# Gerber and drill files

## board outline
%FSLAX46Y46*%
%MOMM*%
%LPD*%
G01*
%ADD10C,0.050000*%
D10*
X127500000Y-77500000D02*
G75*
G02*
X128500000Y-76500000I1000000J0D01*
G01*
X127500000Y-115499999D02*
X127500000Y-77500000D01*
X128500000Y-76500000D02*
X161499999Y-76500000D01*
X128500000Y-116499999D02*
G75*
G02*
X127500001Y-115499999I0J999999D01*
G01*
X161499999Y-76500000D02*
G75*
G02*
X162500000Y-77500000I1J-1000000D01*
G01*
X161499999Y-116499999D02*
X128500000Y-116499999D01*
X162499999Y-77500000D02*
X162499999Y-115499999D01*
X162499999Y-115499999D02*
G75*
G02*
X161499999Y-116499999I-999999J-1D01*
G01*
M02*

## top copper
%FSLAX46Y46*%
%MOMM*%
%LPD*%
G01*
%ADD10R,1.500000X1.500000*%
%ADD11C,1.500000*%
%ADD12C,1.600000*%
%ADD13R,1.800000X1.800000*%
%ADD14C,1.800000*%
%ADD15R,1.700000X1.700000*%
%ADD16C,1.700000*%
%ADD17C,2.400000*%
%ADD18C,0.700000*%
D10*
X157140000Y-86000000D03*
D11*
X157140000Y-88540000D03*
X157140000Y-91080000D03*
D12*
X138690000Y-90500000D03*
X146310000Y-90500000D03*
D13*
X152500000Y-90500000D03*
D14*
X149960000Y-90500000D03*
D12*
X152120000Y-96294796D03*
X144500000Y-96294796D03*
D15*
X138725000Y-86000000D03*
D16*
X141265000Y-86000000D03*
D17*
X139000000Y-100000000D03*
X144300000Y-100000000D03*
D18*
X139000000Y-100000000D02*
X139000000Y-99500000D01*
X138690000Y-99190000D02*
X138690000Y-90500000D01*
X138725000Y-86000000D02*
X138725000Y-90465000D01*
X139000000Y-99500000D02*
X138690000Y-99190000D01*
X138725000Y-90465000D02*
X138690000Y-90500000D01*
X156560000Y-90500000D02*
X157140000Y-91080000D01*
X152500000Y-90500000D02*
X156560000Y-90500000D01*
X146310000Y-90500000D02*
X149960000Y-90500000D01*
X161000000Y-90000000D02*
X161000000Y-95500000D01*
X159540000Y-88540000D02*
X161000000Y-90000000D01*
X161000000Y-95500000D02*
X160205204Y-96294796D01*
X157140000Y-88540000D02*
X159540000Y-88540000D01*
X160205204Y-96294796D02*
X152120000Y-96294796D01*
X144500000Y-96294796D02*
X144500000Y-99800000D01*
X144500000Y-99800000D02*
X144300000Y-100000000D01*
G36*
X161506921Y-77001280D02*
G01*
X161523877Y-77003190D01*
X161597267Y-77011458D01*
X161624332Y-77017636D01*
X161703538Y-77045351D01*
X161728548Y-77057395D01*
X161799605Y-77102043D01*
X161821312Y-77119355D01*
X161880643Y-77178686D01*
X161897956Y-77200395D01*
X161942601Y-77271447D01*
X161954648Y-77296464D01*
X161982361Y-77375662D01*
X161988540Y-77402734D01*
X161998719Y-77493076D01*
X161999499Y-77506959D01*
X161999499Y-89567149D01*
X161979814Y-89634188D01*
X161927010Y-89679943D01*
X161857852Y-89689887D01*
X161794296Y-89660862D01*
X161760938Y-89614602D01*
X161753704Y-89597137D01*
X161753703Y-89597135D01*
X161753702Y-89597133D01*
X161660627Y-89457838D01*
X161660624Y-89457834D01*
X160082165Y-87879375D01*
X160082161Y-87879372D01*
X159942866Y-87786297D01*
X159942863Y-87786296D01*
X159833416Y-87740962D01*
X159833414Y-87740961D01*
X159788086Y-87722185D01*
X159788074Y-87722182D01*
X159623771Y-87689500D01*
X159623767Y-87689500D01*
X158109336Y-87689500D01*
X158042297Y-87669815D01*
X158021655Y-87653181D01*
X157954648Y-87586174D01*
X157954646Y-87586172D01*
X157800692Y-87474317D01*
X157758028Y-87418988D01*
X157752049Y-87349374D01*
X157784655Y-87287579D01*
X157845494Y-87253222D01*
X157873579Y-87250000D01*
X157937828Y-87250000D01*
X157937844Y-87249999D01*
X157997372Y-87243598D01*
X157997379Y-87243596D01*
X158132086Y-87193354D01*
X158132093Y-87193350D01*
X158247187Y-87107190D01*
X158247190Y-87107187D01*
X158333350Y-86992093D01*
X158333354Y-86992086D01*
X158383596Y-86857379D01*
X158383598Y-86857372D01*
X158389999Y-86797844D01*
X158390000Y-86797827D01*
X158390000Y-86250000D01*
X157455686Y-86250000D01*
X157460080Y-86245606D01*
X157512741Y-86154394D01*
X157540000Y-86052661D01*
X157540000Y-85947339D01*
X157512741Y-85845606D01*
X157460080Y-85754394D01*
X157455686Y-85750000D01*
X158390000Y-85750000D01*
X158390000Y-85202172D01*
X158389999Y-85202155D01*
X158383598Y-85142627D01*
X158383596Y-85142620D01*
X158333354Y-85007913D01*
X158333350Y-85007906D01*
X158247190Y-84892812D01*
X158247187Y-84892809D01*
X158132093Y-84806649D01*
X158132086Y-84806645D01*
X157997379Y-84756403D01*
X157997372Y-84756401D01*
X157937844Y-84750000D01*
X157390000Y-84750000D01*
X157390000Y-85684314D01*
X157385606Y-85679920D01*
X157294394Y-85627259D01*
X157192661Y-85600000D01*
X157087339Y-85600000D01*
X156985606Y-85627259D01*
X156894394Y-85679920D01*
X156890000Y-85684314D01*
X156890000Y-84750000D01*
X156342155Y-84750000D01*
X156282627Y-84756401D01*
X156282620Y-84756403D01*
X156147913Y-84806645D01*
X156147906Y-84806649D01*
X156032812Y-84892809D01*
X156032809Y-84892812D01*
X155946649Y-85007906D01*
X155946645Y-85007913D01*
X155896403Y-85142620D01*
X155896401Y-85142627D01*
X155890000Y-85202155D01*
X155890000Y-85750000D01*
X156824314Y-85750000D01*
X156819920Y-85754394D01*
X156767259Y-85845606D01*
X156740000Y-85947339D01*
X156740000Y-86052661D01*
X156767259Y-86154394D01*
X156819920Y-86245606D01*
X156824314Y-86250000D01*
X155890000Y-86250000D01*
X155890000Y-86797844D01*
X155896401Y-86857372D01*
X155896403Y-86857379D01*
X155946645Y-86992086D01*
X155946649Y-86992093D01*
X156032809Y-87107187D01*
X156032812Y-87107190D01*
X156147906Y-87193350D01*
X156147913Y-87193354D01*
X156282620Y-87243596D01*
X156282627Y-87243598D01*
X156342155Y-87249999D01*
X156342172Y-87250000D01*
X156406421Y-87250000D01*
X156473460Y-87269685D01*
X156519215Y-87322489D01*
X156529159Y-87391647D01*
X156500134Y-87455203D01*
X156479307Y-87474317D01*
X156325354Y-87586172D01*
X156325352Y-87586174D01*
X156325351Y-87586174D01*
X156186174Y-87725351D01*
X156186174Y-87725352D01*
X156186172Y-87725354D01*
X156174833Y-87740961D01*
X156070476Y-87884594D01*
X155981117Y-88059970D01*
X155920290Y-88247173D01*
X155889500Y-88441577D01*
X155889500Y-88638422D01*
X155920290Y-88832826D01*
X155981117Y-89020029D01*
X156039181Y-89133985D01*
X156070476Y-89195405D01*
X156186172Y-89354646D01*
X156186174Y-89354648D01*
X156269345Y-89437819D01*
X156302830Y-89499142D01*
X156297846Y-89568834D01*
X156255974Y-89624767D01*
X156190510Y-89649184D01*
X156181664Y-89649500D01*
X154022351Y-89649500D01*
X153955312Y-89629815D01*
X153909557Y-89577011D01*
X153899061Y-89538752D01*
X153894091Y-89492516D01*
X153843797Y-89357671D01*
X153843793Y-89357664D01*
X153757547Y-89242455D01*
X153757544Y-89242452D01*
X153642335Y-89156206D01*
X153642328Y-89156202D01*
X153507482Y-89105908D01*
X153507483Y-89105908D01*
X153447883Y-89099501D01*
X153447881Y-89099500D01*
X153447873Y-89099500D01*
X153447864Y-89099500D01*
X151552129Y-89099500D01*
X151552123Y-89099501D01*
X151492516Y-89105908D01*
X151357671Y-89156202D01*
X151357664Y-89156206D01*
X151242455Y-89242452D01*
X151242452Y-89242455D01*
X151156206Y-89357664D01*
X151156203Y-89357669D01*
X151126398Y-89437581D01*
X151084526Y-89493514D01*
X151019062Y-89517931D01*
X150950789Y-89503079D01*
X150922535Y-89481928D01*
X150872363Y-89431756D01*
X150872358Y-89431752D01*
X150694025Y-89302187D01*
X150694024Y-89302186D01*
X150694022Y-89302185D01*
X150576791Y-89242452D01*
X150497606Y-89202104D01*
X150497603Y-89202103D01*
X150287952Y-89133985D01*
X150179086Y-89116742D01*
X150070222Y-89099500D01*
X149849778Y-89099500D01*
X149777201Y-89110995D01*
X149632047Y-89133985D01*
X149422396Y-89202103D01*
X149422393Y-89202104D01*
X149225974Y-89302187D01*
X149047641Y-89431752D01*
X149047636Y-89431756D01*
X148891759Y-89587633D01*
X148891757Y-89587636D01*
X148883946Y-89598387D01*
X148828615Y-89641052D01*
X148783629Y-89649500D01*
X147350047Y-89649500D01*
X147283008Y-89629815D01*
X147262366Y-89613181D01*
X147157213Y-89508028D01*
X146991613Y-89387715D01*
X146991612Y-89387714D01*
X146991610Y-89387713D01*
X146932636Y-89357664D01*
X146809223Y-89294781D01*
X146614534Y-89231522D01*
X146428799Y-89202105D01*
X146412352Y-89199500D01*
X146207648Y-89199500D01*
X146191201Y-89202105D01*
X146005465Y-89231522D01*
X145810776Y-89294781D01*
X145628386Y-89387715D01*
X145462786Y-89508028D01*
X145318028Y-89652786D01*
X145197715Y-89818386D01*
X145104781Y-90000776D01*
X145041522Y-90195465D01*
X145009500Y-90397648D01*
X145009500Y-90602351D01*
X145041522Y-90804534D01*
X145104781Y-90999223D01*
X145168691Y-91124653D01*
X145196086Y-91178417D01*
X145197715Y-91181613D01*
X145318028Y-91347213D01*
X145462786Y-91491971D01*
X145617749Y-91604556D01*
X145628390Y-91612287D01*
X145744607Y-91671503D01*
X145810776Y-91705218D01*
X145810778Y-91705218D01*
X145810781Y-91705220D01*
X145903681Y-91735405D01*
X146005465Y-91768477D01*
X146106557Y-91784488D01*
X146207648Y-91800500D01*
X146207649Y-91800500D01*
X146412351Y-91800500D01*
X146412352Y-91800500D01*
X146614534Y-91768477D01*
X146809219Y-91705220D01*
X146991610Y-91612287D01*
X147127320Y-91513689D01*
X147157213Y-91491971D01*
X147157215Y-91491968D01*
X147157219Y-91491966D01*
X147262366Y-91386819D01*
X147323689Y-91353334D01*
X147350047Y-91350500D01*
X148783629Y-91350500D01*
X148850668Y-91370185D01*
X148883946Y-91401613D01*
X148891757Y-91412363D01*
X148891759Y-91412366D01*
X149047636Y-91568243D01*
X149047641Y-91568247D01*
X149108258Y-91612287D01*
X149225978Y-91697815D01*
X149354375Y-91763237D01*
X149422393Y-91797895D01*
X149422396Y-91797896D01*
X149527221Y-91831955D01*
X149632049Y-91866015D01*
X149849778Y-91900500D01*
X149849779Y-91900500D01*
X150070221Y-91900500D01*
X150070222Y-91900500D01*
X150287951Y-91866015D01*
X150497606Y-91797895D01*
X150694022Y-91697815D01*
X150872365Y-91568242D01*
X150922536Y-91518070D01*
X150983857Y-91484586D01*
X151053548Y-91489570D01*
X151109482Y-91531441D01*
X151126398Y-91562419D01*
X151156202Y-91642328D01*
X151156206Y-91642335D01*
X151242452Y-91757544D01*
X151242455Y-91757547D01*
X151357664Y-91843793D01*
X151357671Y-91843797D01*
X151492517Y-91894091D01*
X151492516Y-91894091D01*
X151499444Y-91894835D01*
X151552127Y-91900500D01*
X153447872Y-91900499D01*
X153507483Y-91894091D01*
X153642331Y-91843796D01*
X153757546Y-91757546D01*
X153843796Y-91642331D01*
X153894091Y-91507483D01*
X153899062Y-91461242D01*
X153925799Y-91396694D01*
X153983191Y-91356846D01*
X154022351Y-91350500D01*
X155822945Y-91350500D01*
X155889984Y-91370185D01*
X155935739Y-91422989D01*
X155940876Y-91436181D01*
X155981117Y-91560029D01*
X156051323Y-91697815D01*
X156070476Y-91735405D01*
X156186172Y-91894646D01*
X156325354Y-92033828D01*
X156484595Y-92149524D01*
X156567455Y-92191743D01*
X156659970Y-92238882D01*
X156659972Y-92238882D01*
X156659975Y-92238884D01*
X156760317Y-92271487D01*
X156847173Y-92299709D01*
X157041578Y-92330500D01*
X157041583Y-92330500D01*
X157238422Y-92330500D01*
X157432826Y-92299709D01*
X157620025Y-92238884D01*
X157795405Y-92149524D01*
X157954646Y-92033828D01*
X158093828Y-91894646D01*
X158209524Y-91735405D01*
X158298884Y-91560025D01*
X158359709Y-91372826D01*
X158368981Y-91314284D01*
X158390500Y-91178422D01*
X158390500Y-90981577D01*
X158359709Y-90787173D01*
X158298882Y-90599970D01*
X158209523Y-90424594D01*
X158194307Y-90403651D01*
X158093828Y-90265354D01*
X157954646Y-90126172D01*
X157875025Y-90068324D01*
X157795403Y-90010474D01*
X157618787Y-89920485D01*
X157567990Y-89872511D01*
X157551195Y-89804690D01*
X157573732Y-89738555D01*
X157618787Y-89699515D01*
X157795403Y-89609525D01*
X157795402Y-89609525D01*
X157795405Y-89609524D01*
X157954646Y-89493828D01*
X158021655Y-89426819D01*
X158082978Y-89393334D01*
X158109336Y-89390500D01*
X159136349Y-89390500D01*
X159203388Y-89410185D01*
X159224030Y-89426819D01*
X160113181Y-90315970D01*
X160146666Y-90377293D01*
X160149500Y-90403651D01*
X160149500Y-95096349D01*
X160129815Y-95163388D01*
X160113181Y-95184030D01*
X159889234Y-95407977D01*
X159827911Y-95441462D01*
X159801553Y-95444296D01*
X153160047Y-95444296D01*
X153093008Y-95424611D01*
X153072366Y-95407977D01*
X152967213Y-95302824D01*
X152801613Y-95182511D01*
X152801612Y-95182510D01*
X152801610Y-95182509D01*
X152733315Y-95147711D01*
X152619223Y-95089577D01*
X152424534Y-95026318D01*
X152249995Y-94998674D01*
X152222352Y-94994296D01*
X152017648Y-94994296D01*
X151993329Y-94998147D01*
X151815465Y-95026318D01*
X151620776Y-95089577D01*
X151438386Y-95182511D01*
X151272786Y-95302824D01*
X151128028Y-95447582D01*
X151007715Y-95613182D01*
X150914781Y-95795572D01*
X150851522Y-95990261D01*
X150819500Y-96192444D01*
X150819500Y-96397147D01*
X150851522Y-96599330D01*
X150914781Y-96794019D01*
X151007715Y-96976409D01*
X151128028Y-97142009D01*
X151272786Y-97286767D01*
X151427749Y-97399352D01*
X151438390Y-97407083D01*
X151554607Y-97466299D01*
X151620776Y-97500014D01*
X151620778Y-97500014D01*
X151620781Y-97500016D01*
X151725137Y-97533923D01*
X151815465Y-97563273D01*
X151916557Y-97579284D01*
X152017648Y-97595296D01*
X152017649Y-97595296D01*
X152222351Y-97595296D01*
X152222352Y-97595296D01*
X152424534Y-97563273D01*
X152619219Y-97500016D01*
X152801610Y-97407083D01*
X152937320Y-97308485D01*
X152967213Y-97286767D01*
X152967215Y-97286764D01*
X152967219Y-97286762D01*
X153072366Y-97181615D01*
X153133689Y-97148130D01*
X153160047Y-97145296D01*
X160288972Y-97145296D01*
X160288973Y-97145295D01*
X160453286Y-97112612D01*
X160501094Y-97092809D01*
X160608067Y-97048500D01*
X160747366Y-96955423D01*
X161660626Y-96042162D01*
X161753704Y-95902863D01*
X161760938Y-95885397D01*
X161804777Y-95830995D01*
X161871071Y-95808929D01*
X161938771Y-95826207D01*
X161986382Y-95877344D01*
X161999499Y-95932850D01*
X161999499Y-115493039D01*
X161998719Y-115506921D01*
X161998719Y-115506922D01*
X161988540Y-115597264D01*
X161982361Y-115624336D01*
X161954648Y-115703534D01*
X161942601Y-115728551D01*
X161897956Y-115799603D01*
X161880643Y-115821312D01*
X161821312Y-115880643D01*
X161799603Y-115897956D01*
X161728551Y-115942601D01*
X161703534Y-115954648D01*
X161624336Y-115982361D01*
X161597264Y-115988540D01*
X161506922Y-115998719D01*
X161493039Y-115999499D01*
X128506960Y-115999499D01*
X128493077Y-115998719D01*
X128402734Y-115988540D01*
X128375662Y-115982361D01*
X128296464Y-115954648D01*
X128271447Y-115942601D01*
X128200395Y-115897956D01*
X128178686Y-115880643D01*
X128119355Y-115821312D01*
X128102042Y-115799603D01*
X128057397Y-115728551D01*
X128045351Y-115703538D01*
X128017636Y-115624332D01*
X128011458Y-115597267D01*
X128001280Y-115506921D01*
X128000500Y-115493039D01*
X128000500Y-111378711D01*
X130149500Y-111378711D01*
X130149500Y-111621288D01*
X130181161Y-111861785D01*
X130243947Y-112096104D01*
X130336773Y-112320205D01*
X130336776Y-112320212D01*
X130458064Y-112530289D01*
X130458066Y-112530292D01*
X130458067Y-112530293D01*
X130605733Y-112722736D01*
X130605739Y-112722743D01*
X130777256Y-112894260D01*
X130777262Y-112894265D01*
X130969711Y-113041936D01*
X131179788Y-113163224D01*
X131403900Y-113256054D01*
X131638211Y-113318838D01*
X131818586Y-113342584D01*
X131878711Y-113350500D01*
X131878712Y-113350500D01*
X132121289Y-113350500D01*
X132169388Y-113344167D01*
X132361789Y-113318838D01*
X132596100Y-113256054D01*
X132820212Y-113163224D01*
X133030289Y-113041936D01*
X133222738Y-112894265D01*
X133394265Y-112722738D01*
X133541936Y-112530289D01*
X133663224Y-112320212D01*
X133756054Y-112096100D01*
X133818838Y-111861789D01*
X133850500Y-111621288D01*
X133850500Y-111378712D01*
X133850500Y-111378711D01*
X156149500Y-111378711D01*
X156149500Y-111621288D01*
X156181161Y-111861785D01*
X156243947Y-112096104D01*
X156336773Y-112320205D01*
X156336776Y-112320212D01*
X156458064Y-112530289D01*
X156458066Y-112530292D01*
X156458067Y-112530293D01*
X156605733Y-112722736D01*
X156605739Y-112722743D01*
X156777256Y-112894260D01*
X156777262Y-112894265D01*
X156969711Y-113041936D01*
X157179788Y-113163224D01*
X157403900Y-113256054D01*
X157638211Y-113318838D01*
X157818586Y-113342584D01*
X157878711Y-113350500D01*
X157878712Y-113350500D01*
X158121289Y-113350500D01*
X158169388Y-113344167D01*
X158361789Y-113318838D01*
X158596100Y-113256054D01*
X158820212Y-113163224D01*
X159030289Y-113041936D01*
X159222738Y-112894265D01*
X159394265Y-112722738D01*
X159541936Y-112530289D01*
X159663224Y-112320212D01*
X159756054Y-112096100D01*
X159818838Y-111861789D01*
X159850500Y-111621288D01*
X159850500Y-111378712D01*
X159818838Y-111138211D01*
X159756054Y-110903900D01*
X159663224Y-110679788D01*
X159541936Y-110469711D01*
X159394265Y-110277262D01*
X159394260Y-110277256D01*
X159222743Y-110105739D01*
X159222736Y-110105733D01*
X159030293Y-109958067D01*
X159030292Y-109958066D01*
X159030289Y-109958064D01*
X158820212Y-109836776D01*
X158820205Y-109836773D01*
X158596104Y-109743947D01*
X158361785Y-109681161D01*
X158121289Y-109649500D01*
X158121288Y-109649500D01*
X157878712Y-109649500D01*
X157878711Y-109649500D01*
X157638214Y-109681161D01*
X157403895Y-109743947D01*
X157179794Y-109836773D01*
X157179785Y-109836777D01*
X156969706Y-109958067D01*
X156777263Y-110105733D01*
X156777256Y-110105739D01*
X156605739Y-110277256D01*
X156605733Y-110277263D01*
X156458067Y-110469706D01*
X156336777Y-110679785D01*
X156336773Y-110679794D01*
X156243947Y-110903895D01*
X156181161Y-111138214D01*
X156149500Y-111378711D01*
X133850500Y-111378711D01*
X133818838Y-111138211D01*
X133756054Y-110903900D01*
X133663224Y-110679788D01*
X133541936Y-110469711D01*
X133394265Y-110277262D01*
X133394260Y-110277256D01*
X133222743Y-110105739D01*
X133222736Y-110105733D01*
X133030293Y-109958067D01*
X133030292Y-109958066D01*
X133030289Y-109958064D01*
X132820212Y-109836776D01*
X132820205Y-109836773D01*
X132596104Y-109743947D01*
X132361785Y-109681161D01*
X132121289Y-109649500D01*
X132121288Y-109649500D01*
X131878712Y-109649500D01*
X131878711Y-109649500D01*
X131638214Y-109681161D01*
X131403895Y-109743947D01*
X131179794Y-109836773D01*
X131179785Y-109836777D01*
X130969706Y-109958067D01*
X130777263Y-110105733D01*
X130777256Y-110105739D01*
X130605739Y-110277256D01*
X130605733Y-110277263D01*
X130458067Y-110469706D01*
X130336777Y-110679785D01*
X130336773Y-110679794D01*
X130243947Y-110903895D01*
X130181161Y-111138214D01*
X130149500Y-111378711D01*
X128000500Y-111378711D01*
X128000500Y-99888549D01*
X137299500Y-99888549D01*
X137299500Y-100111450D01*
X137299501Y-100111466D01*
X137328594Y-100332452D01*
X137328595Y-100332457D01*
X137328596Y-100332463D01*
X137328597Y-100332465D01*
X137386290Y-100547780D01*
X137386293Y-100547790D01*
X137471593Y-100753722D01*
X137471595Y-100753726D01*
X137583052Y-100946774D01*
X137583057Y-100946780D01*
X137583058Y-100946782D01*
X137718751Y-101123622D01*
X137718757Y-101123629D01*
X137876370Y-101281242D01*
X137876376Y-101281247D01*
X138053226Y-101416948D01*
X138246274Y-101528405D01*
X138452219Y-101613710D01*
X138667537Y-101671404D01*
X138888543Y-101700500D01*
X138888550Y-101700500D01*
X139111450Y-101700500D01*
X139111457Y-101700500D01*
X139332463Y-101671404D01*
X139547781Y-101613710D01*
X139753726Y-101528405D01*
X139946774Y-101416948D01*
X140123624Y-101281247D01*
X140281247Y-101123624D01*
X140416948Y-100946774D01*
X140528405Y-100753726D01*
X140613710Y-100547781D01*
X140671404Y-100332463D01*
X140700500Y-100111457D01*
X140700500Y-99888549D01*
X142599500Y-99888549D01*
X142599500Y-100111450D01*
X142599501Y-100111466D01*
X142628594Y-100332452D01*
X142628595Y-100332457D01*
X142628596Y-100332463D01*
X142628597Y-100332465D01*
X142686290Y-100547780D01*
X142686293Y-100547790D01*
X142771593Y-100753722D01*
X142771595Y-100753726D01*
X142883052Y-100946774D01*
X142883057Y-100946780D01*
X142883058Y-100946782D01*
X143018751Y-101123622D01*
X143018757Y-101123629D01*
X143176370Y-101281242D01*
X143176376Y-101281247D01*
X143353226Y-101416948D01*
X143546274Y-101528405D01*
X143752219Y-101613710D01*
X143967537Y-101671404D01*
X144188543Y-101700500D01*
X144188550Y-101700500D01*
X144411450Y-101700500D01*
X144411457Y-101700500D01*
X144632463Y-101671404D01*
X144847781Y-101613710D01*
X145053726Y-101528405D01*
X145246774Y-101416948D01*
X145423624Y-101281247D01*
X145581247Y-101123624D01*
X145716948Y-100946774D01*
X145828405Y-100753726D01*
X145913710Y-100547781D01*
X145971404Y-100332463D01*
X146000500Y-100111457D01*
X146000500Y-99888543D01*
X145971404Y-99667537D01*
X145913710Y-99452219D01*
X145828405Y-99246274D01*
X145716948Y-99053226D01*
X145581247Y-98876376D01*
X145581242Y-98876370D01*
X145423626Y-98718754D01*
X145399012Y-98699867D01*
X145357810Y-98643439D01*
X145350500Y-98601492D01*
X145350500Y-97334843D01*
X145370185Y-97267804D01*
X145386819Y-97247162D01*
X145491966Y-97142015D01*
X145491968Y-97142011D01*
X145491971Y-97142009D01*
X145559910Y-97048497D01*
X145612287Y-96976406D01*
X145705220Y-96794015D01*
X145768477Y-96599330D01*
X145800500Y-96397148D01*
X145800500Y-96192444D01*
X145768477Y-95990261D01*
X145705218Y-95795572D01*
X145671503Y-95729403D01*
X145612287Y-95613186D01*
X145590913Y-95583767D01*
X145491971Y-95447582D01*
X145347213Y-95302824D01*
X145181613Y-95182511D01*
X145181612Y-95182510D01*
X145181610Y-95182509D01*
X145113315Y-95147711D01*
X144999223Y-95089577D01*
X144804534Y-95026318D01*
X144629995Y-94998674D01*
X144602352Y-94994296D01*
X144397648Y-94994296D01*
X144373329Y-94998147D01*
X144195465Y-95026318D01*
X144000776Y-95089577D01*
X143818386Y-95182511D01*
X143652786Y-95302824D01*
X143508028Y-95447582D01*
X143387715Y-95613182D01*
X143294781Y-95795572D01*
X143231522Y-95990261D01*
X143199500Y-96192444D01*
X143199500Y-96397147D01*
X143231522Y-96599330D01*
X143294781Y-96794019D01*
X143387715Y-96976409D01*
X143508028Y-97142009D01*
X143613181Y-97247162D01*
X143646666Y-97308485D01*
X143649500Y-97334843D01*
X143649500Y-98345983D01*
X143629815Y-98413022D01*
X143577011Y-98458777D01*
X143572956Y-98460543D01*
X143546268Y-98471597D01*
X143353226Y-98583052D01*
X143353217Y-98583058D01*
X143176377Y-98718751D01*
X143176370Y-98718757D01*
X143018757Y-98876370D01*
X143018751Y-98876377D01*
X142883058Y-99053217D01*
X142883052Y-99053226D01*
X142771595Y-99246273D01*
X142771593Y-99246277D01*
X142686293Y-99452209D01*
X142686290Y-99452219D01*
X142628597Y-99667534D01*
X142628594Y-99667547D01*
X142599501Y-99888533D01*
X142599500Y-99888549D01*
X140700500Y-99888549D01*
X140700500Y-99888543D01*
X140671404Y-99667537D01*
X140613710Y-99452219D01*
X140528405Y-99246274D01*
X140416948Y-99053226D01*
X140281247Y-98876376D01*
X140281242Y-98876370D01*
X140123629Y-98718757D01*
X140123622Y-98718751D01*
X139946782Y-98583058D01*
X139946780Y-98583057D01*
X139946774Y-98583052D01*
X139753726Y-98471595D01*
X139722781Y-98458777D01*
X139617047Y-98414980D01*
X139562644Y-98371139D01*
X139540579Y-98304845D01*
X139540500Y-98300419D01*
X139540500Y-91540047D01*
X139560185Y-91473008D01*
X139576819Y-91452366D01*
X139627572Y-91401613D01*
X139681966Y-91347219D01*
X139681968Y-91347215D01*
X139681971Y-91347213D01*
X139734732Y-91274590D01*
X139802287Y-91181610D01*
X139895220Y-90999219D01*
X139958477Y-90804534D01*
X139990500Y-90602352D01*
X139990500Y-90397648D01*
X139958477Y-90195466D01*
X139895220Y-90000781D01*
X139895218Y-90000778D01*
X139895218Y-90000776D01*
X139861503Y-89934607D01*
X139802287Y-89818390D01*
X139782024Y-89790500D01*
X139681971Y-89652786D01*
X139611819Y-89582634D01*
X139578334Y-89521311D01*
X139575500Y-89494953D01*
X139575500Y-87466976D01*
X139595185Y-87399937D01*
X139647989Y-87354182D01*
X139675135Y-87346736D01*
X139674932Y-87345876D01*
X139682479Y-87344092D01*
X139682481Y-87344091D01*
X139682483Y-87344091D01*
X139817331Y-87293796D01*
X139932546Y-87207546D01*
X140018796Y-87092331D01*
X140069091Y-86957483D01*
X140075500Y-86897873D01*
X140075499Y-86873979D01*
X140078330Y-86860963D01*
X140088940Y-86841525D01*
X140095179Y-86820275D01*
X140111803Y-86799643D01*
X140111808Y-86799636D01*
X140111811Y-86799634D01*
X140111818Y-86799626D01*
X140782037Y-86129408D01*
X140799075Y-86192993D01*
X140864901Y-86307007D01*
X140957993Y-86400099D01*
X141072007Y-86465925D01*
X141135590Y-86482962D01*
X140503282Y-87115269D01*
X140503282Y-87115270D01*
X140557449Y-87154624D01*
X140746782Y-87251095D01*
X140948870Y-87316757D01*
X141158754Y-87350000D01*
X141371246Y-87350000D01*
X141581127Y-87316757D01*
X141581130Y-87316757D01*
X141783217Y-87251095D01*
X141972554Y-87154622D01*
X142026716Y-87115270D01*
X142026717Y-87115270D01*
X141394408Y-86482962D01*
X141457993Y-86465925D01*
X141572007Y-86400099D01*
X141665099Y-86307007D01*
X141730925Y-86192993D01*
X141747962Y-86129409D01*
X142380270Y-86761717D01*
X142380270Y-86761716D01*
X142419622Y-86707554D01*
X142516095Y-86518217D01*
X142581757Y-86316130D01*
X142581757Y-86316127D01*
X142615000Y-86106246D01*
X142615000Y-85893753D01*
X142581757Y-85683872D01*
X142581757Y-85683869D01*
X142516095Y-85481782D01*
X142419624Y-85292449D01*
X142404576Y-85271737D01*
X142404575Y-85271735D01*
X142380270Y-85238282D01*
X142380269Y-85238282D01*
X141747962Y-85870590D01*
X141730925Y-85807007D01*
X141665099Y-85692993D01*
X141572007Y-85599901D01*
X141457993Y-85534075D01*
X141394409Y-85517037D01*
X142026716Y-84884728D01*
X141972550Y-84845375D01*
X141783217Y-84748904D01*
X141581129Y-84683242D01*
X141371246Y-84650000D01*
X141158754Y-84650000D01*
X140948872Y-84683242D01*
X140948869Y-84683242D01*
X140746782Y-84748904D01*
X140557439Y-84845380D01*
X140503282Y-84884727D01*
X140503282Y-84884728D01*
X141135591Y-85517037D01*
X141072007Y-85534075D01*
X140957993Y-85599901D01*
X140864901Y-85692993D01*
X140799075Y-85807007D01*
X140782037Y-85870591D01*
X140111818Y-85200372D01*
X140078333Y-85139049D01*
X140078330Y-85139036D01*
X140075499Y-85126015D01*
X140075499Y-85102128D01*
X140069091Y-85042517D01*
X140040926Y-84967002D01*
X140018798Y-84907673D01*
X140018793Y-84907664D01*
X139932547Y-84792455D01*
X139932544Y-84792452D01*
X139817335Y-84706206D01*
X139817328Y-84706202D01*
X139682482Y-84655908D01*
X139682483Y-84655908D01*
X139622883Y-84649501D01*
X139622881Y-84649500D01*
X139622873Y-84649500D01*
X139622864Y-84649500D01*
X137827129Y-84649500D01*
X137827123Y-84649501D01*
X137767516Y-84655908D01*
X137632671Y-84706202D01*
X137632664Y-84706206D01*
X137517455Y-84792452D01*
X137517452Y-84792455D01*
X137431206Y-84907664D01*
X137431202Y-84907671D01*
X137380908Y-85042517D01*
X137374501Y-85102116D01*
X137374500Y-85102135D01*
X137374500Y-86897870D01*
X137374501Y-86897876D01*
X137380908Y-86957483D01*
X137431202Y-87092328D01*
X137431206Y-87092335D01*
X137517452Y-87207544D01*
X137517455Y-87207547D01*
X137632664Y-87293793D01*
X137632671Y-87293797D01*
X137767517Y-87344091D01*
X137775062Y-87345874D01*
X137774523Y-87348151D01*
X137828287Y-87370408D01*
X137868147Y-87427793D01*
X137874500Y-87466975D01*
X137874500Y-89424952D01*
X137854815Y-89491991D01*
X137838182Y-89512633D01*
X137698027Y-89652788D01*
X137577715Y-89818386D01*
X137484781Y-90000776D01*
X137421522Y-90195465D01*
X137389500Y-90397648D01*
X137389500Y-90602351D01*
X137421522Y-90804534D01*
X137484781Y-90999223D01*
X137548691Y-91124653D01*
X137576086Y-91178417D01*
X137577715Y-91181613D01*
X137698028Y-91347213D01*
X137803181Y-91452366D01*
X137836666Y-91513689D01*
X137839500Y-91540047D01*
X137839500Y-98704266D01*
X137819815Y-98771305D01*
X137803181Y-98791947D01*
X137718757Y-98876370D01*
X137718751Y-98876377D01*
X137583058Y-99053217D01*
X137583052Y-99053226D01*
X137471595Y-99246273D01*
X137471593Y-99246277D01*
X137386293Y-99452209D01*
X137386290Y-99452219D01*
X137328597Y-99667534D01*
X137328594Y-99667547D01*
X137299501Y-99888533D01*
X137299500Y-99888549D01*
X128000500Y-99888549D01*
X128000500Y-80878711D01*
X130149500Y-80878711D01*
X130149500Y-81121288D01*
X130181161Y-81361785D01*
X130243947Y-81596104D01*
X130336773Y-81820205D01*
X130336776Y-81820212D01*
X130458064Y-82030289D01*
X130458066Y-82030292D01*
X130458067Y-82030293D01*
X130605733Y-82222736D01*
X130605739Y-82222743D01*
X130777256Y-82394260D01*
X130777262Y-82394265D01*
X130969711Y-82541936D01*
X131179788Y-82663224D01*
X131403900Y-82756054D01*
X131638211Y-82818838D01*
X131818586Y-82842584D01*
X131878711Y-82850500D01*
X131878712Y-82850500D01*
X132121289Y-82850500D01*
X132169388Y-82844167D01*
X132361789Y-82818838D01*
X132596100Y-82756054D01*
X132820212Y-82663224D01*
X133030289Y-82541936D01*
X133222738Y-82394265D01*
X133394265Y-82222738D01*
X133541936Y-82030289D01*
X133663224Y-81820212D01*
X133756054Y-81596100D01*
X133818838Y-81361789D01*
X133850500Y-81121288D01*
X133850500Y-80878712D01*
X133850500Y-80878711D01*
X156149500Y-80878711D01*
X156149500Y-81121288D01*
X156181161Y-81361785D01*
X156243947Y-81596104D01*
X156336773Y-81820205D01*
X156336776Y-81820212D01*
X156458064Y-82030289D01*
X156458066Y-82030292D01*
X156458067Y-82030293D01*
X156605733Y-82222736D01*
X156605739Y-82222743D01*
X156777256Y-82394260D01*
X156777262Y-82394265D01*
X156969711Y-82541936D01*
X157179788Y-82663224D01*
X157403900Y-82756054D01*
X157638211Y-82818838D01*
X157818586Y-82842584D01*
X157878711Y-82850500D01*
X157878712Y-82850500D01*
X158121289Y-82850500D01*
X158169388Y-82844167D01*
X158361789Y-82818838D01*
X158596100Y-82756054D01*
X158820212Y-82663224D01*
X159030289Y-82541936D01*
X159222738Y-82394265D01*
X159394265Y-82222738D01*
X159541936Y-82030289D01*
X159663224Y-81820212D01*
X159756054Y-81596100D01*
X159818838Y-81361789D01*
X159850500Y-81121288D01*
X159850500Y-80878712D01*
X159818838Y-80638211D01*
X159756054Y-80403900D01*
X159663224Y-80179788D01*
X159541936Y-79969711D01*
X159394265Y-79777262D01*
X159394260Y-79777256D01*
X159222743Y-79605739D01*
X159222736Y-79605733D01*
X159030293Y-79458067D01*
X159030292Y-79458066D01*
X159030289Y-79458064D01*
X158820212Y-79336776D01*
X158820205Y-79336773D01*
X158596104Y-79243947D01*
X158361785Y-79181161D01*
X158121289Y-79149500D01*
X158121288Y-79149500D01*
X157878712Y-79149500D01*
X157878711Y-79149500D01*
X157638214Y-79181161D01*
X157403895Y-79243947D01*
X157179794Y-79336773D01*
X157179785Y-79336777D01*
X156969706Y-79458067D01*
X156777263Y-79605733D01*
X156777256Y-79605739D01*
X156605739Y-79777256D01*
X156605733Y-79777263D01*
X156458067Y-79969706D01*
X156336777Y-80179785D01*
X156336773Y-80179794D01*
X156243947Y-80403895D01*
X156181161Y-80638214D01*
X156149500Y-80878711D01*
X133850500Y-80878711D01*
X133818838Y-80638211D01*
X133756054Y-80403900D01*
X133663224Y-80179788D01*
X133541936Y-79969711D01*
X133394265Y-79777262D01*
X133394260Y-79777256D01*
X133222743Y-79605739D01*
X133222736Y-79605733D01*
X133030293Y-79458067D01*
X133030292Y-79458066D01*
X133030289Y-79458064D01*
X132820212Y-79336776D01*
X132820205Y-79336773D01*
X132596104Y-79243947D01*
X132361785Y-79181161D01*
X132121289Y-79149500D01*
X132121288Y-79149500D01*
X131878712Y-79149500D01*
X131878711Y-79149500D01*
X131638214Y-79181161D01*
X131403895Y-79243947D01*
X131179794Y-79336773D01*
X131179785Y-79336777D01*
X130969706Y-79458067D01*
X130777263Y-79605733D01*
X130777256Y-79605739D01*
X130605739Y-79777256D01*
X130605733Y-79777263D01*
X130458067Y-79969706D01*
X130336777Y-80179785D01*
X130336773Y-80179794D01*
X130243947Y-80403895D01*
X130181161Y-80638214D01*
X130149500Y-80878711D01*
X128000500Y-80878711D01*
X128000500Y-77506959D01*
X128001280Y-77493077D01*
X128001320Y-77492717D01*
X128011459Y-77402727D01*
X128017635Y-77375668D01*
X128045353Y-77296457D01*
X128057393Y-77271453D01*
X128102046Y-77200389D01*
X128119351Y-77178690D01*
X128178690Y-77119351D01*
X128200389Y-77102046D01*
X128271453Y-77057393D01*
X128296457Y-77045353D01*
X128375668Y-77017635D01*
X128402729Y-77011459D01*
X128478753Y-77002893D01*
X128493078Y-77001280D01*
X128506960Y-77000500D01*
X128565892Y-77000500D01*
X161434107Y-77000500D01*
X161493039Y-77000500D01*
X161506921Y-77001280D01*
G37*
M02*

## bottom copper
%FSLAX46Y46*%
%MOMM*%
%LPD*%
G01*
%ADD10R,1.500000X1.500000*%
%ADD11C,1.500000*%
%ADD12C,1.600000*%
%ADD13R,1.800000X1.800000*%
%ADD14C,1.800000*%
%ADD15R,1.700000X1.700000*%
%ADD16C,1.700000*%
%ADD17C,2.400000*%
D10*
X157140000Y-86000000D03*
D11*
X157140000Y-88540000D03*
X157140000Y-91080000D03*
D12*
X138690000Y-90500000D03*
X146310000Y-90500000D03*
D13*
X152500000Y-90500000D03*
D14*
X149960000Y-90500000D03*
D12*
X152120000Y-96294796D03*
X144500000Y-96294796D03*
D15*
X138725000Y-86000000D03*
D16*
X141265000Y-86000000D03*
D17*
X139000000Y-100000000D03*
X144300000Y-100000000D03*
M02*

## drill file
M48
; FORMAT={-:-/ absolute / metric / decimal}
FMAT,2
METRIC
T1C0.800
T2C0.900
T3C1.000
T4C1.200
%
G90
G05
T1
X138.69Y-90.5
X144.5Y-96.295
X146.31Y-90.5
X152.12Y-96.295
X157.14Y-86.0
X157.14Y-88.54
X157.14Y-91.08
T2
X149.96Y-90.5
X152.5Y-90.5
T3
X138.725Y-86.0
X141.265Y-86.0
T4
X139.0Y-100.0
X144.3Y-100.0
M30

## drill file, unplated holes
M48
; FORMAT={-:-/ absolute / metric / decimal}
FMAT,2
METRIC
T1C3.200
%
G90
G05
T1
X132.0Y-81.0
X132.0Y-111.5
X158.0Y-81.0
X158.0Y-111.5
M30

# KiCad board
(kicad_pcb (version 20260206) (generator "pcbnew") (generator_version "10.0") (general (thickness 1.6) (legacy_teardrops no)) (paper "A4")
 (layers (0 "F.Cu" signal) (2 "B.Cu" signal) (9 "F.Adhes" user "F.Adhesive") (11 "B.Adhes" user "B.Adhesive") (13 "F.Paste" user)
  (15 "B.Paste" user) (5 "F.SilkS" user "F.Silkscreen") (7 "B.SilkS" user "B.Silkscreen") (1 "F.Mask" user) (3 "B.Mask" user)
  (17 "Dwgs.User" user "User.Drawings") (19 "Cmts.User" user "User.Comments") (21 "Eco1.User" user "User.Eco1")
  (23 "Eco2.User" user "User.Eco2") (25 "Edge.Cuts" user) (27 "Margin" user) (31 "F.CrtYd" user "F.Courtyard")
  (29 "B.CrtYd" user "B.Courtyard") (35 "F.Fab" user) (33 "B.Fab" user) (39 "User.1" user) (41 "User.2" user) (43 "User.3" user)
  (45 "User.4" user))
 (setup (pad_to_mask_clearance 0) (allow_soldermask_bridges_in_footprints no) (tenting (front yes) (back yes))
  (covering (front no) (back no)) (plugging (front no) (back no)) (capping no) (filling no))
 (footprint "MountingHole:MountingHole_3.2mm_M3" (layer "F.Cu") (at 132 81)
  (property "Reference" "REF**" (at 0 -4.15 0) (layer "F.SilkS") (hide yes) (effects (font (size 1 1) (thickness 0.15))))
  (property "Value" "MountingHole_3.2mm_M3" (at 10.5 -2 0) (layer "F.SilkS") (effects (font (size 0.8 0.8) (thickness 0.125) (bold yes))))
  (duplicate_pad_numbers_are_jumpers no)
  (pad "" np_thru_hole circle (at 0 0) (size 3.2 3.2) (drill 3.2) (layers "*.Cu" "*.Mask")))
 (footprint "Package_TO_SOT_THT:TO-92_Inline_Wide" (layer "F.Cu") (at 157.14 86 -90)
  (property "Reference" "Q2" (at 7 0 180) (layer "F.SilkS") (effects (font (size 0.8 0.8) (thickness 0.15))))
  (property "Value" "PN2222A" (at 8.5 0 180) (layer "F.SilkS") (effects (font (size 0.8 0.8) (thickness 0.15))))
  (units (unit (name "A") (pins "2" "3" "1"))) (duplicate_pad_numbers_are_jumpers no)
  (pad "1" thru_hole rect (at 0 0 270) (size 1.5 1.5) (drill 0.8) (layers "*.Cu" "*.Mask") (remove_unused_layers no) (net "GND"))
  (pad "2" thru_hole circle (at 2.54 0 270) (size 1.5 1.5) (drill 0.8) (layers "*.Cu" "*.Mask") (remove_unused_layers no) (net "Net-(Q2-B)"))
  (pad "3" thru_hole circle (at 5.08 0 270) (size 1.5 1.5) (drill 0.8) (layers "*.Cu" "*.Mask") (remove_unused_layers no) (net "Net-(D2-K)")))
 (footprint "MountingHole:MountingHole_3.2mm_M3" (layer "F.Cu") (at 158 81)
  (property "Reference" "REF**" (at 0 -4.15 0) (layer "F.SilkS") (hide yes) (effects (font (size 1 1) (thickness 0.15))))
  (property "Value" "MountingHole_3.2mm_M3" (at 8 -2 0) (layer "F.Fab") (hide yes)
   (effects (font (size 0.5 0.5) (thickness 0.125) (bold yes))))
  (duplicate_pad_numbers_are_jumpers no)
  (pad "" np_thru_hole circle (at 0 0) (size 3.2 3.2) (drill 3.2) (layers "*.Cu" "*.Mask")))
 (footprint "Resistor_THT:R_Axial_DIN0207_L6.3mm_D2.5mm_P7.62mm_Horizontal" (layer "F.Cu") (at 138.69 90.5)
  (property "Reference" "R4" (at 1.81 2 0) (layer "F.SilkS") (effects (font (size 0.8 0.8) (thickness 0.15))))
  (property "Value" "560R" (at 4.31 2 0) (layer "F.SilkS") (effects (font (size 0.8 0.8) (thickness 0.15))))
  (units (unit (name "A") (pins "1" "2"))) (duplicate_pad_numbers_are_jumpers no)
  (pad "1" thru_hole circle (at 0 0) (size 1.6 1.6) (drill 0.8) (layers "*.Cu" "*.Mask") (remove_unused_layers no) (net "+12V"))
  (pad "2" thru_hole circle (at 7.62 0) (size 1.6 1.6) (drill 0.8) (layers "*.Cu" "*.Mask") (remove_unused_layers no) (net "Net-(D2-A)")))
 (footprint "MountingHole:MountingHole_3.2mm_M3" (layer "F.Cu") (at 158 111.5)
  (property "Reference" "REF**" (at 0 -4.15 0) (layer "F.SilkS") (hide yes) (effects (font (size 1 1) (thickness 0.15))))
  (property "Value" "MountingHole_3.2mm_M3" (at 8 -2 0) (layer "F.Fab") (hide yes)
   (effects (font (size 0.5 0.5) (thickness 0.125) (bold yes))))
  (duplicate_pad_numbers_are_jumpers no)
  (pad "" np_thru_hole circle (at 0 0) (size 3.2 3.2) (drill 3.2) (layers "*.Cu" "*.Mask")))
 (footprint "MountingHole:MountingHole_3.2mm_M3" (layer "F.Cu") (at 132 111.5)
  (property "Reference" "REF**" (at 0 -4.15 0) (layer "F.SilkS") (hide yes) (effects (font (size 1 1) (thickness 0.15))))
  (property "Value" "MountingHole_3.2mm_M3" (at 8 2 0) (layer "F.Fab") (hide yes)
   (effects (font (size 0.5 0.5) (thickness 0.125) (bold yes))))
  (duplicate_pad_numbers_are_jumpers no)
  (pad "" np_thru_hole circle (at 0 0) (size 3.2 3.2) (drill 3.2) (layers "*.Cu" "*.Mask")))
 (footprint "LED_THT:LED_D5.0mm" (layer "F.Cu") (at 152.5 90.5 180)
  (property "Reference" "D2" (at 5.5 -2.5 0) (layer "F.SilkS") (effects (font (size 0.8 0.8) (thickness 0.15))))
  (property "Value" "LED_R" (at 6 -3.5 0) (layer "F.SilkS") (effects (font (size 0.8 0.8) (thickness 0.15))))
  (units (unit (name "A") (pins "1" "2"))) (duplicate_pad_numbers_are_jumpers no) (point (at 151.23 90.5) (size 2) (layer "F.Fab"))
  (pad "1" thru_hole rect (at 0 0 180) (size 1.8 1.8) (drill 0.9) (layers "*.Cu" "*.Mask") (remove_unused_layers no) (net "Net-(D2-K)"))
  (pad "2" thru_hole circle (at 2.54 0 180) (size 1.8 1.8) (drill 0.9) (layers "*.Cu" "*.Mask") (remove_unused_layers no) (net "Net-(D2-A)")))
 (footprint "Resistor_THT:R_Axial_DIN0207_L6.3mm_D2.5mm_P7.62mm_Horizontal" (layer "F.Cu") (at 152.12 96.294796 180)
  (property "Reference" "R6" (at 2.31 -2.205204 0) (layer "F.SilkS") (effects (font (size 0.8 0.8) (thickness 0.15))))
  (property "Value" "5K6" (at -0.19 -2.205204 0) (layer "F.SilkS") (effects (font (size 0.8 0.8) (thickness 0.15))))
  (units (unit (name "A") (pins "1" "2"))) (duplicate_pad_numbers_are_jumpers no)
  (pad "1" thru_hole circle (at 0 0 180) (size 1.6 1.6) (drill 0.8) (layers "*.Cu" "*.Mask") (remove_unused_layers no) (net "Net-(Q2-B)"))
  (pad "2" thru_hole circle (at 7.62 0 180) (size 1.6 1.6) (drill 0.8) (layers "*.Cu" "*.Mask") (remove_unused_layers no)
   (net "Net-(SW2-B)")))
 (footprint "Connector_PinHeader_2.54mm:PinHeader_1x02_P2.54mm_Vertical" (layer "F.Cu") (at 138.725 86 90)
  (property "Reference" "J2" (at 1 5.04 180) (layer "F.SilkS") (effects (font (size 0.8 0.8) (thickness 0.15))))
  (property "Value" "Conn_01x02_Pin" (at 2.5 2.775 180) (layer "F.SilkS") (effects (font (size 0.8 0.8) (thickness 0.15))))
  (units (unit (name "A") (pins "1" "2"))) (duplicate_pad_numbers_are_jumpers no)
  (pad "1" thru_hole rect (at 0 0 90) (size 1.7 1.7) (drill 1) (layers "*.Cu" "*.Mask") (remove_unused_layers no) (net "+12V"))
  (pad "2" thru_hole circle (at 0 2.54 90) (size 1.7 1.7) (drill 1) (layers "*.Cu" "*.Mask") (remove_unused_layers no) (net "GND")))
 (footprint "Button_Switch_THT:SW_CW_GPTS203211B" (layer "B.Cu") (at 139 100 -90)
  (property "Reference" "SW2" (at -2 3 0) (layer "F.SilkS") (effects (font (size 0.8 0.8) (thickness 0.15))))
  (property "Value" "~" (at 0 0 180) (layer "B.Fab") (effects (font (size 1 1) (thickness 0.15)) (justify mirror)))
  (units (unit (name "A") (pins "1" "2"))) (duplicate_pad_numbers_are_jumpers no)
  (pad "1" thru_hole circle (at 0 0 270) (size 2.4 2.4) (drill 1.2) (layers "*.Cu" "*.Mask") (remove_unused_layers no) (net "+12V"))
  (pad "2" thru_hole circle (at 0 -5.3 270) (size 2.4 2.4) (drill 1.2) (layers "*.Cu" "*.Mask") (remove_unused_layers no)
   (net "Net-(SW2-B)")))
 (gr_arc (start 127.5 77.5) (mid 127.792893 76.792893) (end 128.5 76.5) (stroke (width 0.05) (type default)) (layer "Edge.Cuts"))
 (gr_line (start 127.5 115.499999) (end 127.5 77.5) (stroke (width 0.05) (type default)) (layer "Edge.Cuts"))
 (gr_line (start 128.5 76.5) (end 161.499999 76.5) (stroke (width 0.05) (type default)) (layer "Edge.Cuts"))
 (gr_arc (start 128.5 116.499999) (mid 127.792893 116.207106) (end 127.5 115.499999) (stroke (width 0.05) (type default))
  (layer "Edge.Cuts"))
 (gr_arc (start 161.499999 76.5) (mid 162.207106 76.792893) (end 162.499999 77.5) (stroke (width 0.05) (type default)) (layer "Edge.Cuts"))
 (gr_line (start 161.499999 116.499999) (end 128.5 116.499999) (stroke (width 0.05) (type default)) (layer "Edge.Cuts"))
 (gr_line (start 162.499999 77.5) (end 162.499999 115.499999) (stroke (width 0.05) (type default)) (layer "Edge.Cuts"))
 (gr_arc (start 162.499999 115.499999) (mid 162.207106 116.207106) (end 161.499999 116.499999) (stroke (width 0.05) (type default))
  (layer "Edge.Cuts"))
 (segment (start 161 90) (end 161 95.5) (width 0.7) (layer "F.Cu") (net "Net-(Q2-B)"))
 (segment (start 159.54 88.54) (end 161 90) (width 0.7) (layer "F.Cu") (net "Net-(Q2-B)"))
 (segment (start 161 95.5) (end 160.205204 96.294796) (width 0.7) (layer "F.Cu") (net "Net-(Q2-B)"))
 (segment (start 157.14 88.54) (end 159.54 88.54) (width 0.7) (layer "F.Cu") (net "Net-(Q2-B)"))
 (segment (start 160.205204 96.294796) (end 152.12 96.294796) (width 0.7) (layer "F.Cu") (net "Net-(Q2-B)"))
 (segment (start 156.56 90.5) (end 157.14 91.08) (width 0.7) (layer "F.Cu") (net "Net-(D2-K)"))
 (segment (start 152.5 90.5) (end 156.56 90.5) (width 0.7) (layer "F.Cu") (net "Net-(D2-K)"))
 (segment (start 139 100) (end 139 99.5) (width 0.7) (layer "F.Cu") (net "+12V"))
 (segment (start 138.69 99.19) (end 138.69 90.5) (width 0.7) (layer "F.Cu") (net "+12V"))
 (segment (start 138.725 86) (end 138.725 90.465) (width 0.7) (layer "F.Cu") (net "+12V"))
 (segment (start 139 99.5) (end 138.69 99.19) (width 0.7) (layer "F.Cu") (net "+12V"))
 (segment (start 138.725 90.465) (end 138.69 90.5) (width 0.7) (layer "F.Cu") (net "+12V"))
 (segment (start 146.31 90.5) (end 149.96 90.5) (width 0.7) (layer "F.Cu") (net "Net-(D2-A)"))
 (segment (start 144.5 96.294796) (end 144.5 99.8) (width 0.7) (layer "F.Cu") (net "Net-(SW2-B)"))
 (segment (start 144.5 99.8) (end 144.3 100) (width 0.7) (layer "F.Cu") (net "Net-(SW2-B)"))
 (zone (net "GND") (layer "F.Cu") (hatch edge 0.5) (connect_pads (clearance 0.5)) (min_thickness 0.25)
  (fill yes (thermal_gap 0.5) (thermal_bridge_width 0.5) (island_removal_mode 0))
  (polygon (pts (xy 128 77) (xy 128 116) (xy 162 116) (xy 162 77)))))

